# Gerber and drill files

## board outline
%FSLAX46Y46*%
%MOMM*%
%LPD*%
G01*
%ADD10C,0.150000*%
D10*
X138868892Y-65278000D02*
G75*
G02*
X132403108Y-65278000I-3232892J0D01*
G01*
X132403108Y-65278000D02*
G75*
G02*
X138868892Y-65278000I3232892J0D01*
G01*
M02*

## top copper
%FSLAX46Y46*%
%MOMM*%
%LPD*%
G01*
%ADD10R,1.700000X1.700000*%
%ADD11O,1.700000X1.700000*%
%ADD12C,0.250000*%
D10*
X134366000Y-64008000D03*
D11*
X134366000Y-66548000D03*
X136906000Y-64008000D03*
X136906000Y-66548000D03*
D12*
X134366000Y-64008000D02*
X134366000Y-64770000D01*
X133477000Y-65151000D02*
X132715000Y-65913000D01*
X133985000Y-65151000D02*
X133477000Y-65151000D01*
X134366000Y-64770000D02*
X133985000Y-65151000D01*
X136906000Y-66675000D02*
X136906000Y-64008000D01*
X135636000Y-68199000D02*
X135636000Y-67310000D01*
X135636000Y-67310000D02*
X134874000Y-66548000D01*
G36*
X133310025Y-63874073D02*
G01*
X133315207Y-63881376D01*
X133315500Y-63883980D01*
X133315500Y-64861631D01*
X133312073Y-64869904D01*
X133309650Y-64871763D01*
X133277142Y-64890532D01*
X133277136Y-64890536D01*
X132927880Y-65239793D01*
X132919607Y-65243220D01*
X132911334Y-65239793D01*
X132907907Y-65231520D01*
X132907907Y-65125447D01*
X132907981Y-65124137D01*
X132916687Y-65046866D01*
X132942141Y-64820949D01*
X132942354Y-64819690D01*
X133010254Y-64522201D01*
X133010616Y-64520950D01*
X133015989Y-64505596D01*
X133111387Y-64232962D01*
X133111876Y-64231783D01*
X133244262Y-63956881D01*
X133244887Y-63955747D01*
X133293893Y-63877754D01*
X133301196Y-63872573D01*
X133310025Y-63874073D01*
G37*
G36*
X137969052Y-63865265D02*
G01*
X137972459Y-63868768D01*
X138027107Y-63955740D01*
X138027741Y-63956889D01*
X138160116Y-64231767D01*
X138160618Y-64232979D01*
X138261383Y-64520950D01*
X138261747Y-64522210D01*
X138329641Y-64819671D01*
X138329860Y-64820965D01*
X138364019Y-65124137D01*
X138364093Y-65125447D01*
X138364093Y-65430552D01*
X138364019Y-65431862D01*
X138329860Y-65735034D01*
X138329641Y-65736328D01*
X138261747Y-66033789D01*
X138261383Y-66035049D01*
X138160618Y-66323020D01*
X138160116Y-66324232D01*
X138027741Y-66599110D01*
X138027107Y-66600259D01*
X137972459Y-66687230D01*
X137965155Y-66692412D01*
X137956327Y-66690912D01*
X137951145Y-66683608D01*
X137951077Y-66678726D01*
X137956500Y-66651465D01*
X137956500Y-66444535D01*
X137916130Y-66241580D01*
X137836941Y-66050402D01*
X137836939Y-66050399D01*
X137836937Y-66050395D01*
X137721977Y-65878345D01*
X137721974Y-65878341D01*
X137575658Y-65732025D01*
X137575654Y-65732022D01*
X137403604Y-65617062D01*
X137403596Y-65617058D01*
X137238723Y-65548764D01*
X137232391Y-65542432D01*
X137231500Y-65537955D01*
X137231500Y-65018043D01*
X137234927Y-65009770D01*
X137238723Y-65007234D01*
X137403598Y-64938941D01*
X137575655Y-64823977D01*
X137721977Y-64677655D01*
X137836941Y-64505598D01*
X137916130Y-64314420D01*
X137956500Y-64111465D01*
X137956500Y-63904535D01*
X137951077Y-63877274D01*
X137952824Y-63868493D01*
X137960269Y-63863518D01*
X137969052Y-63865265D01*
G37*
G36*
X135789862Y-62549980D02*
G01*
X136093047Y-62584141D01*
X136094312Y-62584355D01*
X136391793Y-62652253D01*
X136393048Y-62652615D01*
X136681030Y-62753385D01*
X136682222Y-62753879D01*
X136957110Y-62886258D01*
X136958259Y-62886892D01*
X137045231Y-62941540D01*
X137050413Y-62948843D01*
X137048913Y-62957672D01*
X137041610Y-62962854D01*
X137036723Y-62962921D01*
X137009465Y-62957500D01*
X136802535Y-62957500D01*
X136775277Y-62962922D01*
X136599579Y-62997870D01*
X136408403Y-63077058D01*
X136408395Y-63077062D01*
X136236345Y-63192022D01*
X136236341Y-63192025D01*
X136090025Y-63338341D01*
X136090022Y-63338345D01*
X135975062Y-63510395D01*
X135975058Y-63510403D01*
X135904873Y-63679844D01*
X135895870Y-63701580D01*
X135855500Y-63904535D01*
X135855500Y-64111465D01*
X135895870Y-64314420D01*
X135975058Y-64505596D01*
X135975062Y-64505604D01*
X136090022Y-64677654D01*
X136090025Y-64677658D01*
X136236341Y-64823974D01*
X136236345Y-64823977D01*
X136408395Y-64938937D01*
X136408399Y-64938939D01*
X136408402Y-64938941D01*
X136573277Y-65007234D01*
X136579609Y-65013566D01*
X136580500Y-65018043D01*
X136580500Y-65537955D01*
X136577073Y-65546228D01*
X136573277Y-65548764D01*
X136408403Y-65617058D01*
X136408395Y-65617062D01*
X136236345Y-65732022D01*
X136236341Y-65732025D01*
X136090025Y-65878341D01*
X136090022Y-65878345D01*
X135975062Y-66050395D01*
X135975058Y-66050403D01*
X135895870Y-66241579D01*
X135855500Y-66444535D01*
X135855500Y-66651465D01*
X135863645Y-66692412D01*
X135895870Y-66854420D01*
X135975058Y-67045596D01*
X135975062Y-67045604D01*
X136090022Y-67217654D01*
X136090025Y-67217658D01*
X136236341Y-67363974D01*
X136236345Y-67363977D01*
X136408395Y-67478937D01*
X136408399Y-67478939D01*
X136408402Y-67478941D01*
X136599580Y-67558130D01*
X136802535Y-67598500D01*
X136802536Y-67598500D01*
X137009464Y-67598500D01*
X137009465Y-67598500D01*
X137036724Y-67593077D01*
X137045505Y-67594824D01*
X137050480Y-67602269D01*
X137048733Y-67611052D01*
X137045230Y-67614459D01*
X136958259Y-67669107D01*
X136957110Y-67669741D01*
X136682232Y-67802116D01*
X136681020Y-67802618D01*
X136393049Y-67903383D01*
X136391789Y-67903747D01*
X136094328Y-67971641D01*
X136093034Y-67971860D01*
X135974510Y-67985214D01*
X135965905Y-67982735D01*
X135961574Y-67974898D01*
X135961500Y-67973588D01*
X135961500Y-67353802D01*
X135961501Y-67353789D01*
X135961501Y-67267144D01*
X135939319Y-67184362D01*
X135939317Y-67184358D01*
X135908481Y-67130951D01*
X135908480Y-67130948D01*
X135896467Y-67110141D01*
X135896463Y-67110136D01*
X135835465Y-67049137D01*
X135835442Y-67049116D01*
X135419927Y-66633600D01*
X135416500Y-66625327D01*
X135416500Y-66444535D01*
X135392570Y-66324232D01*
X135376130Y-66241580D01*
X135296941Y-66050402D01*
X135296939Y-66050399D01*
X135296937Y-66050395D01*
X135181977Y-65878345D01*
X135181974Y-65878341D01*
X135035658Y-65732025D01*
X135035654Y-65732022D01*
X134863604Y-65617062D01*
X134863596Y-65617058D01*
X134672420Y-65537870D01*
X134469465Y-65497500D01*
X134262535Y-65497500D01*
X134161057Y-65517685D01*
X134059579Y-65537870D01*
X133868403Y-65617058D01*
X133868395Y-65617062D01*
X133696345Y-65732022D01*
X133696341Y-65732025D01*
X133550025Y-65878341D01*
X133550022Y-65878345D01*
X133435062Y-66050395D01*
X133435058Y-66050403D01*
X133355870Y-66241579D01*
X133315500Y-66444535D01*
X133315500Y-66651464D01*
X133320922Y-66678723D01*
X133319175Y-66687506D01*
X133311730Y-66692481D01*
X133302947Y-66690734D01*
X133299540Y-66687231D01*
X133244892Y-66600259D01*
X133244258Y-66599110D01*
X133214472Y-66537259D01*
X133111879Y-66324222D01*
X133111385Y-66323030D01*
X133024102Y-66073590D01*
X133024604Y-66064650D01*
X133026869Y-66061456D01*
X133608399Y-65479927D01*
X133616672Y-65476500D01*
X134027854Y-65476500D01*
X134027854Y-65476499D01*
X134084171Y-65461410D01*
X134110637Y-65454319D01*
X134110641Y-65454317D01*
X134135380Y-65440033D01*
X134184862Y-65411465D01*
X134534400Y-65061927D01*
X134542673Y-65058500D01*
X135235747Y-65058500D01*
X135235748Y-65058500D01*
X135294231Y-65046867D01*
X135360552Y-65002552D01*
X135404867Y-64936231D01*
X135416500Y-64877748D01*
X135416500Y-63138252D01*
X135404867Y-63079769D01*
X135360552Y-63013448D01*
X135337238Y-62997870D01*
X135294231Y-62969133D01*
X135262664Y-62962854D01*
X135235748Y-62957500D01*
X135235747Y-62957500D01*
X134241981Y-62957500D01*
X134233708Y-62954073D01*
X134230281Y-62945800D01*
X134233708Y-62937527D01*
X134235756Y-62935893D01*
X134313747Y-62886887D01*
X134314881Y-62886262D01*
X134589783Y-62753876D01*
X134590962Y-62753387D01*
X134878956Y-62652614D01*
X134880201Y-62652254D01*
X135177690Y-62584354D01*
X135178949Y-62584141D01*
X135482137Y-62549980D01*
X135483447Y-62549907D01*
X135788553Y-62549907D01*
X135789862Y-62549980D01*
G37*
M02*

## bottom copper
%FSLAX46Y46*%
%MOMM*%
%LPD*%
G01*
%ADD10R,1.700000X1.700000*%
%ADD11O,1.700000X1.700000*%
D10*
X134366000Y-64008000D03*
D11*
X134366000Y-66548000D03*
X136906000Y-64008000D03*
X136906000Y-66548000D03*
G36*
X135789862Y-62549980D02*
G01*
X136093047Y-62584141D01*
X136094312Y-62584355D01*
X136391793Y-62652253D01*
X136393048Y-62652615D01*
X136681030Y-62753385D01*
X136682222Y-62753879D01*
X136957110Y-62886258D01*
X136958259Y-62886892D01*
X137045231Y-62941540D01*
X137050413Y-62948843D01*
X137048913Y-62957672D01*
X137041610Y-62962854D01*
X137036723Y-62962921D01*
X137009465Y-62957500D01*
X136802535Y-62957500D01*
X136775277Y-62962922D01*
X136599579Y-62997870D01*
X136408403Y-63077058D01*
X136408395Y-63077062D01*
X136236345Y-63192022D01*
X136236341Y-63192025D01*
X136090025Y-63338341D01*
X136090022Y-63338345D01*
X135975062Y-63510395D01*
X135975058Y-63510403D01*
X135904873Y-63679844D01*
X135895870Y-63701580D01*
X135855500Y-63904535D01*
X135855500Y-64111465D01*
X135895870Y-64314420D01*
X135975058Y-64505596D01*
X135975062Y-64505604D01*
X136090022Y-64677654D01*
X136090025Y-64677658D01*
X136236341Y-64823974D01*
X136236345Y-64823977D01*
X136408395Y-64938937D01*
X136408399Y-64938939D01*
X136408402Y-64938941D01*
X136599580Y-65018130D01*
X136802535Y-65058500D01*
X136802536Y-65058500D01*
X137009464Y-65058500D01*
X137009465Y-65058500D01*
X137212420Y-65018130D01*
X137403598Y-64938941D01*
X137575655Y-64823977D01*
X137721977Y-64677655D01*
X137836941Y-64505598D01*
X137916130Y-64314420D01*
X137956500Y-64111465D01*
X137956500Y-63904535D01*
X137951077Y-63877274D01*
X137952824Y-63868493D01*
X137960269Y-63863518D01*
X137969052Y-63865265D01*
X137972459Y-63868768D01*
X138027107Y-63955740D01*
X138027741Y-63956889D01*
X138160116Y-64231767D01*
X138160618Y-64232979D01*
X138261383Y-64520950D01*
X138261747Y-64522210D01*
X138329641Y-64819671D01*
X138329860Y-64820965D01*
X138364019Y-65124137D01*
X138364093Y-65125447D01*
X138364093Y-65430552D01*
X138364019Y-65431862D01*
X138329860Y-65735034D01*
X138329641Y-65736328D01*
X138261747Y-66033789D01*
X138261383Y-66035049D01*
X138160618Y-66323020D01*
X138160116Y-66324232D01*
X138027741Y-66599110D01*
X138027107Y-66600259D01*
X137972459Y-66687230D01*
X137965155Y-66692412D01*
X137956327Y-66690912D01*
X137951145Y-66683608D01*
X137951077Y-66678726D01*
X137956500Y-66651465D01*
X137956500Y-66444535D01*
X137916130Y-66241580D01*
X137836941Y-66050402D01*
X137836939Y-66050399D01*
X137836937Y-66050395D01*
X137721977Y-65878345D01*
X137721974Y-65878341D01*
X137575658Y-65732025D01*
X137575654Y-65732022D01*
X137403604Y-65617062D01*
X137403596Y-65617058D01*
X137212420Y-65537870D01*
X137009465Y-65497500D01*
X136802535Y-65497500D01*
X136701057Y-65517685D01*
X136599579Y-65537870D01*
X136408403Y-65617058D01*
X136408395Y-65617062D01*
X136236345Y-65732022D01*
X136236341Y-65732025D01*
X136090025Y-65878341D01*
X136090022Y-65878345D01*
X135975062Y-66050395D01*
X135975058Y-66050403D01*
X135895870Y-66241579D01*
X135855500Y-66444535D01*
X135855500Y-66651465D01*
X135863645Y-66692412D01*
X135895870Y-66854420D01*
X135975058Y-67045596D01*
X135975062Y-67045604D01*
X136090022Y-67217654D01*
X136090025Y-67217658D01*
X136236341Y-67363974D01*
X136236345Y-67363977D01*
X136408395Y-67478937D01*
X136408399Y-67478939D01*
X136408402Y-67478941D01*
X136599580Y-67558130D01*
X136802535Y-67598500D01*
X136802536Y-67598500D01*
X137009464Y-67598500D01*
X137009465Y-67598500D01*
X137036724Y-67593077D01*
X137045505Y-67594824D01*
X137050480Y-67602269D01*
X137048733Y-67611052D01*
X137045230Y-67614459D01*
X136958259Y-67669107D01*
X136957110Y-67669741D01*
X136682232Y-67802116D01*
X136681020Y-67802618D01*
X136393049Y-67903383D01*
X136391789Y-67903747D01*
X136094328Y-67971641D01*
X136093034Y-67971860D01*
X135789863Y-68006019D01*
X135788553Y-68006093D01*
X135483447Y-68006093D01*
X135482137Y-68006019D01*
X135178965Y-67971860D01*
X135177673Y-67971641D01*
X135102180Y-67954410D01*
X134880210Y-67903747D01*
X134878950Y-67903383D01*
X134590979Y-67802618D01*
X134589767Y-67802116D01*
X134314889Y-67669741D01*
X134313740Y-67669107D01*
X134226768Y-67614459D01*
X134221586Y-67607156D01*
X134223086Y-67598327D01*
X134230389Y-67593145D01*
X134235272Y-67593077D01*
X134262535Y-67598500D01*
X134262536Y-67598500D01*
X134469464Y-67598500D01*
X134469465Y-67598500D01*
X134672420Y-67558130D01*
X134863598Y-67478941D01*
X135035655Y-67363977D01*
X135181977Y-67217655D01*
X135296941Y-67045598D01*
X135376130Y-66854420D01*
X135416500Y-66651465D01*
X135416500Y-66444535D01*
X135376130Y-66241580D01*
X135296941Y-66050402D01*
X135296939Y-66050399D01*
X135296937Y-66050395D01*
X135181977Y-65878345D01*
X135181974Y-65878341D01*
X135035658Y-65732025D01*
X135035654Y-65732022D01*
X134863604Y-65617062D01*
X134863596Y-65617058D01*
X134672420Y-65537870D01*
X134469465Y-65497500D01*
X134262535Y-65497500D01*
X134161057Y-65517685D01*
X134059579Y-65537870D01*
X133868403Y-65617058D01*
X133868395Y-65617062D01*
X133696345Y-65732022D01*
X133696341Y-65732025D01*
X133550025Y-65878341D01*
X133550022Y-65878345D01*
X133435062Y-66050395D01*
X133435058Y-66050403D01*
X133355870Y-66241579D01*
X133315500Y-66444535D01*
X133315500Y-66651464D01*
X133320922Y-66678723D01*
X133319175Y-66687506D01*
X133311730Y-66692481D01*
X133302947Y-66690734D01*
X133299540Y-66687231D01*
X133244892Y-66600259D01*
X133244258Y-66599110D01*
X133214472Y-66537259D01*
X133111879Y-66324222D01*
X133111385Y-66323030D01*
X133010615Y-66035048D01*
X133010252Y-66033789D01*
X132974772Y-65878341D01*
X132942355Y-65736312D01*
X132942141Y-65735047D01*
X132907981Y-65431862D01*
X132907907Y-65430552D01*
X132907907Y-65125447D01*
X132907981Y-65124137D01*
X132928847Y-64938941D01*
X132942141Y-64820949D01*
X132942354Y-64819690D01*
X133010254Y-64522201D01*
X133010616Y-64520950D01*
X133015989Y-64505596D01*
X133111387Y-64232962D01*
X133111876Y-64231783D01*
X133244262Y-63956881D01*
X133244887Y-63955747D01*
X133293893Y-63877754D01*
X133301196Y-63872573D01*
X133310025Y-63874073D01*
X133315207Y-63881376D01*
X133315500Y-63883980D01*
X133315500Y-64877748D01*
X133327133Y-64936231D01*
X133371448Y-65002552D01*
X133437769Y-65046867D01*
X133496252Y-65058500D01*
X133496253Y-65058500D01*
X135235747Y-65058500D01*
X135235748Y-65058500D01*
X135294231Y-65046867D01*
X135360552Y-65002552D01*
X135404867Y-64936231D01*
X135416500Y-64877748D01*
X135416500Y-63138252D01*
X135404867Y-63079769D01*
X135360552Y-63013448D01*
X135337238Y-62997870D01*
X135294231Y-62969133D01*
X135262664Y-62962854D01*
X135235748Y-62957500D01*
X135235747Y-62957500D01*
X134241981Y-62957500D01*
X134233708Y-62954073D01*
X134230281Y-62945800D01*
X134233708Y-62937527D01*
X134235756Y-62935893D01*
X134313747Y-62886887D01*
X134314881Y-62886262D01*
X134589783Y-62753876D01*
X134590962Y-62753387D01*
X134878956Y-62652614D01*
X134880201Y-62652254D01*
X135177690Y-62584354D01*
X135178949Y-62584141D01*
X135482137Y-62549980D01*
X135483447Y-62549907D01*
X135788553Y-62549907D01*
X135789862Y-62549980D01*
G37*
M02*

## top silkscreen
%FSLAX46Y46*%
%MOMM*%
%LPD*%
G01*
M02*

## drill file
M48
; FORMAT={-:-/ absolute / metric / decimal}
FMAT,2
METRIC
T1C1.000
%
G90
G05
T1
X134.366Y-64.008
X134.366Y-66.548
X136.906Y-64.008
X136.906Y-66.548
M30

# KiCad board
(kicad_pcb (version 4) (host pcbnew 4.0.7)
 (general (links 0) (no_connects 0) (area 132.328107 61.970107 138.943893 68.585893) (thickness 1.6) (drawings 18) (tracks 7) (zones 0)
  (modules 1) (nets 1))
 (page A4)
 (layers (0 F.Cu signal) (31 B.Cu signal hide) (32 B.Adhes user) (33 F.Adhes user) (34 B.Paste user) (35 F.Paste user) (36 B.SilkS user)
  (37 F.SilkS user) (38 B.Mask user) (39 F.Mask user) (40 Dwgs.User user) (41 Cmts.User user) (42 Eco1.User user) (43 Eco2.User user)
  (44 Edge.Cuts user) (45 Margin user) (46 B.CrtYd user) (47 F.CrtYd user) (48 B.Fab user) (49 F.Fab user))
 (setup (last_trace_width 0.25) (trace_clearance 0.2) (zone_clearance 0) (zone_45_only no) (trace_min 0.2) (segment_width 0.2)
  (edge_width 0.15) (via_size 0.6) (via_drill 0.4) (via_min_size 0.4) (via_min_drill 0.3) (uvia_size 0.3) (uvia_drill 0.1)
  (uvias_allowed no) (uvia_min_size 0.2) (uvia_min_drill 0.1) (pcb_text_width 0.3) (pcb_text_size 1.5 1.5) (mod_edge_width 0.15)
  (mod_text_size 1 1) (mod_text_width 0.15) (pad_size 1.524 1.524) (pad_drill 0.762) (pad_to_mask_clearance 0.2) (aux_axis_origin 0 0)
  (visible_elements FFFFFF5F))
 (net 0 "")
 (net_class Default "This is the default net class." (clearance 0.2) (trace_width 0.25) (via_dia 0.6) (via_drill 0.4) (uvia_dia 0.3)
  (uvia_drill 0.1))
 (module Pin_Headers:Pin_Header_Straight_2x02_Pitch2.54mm (layer B.Cu) (at 134.366 64.008 270)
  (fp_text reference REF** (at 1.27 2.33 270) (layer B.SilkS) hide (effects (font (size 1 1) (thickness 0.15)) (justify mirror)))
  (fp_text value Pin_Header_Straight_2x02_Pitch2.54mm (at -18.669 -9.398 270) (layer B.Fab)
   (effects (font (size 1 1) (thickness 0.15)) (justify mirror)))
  (pad 1 thru_hole rect (at 0 0 270) (size 1.7 1.7) (drill 1) (layers *.Cu *.Mask))
  (pad 2 thru_hole oval (at 2.54 0 270) (size 1.7 1.7) (drill 1) (layers *.Cu *.Mask))
  (pad 3 thru_hole oval (at 0 -2.54 270) (size 1.7 1.7) (drill 1) (layers *.Cu *.Mask))
  (pad 4 thru_hole oval (at 2.54 -2.54 270) (size 1.7 1.7) (drill 1) (layers *.Cu *.Mask)))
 (gr_circle (center 135.636 65.278) (end 133.35 62.992) (layer Edge.Cuts) (width 0.15))
 (segment (start 134.366 64.008) (end 134.366 64.77) (width 0.25) (layer F.Cu) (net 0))
 (segment (start 133.477 65.151) (end 132.715 65.913) (width 0.25) (layer F.Cu) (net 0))
 (segment (start 133.985 65.151) (end 133.477 65.151) (width 0.25) (layer F.Cu) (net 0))
 (segment (start 134.366 64.77) (end 133.985 65.151) (width 0.25) (layer F.Cu) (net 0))
 (segment (start 136.906 66.675) (end 136.906 64.008) (width 0.25) (layer F.Cu) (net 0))
 (segment (start 135.636 68.199) (end 135.636 67.31) (width 0.25) (layer F.Cu) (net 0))
 (segment (start 135.636 67.31) (end 134.874 66.548) (width 0.25) (layer F.Cu) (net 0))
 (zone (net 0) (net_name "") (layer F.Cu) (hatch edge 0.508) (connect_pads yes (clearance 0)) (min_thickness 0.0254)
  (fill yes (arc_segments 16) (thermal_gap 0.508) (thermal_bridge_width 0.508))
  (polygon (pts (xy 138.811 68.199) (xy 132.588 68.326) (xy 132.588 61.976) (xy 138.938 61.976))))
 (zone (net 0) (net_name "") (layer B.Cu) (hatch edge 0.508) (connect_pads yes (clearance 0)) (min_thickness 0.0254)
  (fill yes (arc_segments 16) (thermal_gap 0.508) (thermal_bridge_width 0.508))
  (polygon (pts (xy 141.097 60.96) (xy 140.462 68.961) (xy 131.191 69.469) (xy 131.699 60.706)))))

